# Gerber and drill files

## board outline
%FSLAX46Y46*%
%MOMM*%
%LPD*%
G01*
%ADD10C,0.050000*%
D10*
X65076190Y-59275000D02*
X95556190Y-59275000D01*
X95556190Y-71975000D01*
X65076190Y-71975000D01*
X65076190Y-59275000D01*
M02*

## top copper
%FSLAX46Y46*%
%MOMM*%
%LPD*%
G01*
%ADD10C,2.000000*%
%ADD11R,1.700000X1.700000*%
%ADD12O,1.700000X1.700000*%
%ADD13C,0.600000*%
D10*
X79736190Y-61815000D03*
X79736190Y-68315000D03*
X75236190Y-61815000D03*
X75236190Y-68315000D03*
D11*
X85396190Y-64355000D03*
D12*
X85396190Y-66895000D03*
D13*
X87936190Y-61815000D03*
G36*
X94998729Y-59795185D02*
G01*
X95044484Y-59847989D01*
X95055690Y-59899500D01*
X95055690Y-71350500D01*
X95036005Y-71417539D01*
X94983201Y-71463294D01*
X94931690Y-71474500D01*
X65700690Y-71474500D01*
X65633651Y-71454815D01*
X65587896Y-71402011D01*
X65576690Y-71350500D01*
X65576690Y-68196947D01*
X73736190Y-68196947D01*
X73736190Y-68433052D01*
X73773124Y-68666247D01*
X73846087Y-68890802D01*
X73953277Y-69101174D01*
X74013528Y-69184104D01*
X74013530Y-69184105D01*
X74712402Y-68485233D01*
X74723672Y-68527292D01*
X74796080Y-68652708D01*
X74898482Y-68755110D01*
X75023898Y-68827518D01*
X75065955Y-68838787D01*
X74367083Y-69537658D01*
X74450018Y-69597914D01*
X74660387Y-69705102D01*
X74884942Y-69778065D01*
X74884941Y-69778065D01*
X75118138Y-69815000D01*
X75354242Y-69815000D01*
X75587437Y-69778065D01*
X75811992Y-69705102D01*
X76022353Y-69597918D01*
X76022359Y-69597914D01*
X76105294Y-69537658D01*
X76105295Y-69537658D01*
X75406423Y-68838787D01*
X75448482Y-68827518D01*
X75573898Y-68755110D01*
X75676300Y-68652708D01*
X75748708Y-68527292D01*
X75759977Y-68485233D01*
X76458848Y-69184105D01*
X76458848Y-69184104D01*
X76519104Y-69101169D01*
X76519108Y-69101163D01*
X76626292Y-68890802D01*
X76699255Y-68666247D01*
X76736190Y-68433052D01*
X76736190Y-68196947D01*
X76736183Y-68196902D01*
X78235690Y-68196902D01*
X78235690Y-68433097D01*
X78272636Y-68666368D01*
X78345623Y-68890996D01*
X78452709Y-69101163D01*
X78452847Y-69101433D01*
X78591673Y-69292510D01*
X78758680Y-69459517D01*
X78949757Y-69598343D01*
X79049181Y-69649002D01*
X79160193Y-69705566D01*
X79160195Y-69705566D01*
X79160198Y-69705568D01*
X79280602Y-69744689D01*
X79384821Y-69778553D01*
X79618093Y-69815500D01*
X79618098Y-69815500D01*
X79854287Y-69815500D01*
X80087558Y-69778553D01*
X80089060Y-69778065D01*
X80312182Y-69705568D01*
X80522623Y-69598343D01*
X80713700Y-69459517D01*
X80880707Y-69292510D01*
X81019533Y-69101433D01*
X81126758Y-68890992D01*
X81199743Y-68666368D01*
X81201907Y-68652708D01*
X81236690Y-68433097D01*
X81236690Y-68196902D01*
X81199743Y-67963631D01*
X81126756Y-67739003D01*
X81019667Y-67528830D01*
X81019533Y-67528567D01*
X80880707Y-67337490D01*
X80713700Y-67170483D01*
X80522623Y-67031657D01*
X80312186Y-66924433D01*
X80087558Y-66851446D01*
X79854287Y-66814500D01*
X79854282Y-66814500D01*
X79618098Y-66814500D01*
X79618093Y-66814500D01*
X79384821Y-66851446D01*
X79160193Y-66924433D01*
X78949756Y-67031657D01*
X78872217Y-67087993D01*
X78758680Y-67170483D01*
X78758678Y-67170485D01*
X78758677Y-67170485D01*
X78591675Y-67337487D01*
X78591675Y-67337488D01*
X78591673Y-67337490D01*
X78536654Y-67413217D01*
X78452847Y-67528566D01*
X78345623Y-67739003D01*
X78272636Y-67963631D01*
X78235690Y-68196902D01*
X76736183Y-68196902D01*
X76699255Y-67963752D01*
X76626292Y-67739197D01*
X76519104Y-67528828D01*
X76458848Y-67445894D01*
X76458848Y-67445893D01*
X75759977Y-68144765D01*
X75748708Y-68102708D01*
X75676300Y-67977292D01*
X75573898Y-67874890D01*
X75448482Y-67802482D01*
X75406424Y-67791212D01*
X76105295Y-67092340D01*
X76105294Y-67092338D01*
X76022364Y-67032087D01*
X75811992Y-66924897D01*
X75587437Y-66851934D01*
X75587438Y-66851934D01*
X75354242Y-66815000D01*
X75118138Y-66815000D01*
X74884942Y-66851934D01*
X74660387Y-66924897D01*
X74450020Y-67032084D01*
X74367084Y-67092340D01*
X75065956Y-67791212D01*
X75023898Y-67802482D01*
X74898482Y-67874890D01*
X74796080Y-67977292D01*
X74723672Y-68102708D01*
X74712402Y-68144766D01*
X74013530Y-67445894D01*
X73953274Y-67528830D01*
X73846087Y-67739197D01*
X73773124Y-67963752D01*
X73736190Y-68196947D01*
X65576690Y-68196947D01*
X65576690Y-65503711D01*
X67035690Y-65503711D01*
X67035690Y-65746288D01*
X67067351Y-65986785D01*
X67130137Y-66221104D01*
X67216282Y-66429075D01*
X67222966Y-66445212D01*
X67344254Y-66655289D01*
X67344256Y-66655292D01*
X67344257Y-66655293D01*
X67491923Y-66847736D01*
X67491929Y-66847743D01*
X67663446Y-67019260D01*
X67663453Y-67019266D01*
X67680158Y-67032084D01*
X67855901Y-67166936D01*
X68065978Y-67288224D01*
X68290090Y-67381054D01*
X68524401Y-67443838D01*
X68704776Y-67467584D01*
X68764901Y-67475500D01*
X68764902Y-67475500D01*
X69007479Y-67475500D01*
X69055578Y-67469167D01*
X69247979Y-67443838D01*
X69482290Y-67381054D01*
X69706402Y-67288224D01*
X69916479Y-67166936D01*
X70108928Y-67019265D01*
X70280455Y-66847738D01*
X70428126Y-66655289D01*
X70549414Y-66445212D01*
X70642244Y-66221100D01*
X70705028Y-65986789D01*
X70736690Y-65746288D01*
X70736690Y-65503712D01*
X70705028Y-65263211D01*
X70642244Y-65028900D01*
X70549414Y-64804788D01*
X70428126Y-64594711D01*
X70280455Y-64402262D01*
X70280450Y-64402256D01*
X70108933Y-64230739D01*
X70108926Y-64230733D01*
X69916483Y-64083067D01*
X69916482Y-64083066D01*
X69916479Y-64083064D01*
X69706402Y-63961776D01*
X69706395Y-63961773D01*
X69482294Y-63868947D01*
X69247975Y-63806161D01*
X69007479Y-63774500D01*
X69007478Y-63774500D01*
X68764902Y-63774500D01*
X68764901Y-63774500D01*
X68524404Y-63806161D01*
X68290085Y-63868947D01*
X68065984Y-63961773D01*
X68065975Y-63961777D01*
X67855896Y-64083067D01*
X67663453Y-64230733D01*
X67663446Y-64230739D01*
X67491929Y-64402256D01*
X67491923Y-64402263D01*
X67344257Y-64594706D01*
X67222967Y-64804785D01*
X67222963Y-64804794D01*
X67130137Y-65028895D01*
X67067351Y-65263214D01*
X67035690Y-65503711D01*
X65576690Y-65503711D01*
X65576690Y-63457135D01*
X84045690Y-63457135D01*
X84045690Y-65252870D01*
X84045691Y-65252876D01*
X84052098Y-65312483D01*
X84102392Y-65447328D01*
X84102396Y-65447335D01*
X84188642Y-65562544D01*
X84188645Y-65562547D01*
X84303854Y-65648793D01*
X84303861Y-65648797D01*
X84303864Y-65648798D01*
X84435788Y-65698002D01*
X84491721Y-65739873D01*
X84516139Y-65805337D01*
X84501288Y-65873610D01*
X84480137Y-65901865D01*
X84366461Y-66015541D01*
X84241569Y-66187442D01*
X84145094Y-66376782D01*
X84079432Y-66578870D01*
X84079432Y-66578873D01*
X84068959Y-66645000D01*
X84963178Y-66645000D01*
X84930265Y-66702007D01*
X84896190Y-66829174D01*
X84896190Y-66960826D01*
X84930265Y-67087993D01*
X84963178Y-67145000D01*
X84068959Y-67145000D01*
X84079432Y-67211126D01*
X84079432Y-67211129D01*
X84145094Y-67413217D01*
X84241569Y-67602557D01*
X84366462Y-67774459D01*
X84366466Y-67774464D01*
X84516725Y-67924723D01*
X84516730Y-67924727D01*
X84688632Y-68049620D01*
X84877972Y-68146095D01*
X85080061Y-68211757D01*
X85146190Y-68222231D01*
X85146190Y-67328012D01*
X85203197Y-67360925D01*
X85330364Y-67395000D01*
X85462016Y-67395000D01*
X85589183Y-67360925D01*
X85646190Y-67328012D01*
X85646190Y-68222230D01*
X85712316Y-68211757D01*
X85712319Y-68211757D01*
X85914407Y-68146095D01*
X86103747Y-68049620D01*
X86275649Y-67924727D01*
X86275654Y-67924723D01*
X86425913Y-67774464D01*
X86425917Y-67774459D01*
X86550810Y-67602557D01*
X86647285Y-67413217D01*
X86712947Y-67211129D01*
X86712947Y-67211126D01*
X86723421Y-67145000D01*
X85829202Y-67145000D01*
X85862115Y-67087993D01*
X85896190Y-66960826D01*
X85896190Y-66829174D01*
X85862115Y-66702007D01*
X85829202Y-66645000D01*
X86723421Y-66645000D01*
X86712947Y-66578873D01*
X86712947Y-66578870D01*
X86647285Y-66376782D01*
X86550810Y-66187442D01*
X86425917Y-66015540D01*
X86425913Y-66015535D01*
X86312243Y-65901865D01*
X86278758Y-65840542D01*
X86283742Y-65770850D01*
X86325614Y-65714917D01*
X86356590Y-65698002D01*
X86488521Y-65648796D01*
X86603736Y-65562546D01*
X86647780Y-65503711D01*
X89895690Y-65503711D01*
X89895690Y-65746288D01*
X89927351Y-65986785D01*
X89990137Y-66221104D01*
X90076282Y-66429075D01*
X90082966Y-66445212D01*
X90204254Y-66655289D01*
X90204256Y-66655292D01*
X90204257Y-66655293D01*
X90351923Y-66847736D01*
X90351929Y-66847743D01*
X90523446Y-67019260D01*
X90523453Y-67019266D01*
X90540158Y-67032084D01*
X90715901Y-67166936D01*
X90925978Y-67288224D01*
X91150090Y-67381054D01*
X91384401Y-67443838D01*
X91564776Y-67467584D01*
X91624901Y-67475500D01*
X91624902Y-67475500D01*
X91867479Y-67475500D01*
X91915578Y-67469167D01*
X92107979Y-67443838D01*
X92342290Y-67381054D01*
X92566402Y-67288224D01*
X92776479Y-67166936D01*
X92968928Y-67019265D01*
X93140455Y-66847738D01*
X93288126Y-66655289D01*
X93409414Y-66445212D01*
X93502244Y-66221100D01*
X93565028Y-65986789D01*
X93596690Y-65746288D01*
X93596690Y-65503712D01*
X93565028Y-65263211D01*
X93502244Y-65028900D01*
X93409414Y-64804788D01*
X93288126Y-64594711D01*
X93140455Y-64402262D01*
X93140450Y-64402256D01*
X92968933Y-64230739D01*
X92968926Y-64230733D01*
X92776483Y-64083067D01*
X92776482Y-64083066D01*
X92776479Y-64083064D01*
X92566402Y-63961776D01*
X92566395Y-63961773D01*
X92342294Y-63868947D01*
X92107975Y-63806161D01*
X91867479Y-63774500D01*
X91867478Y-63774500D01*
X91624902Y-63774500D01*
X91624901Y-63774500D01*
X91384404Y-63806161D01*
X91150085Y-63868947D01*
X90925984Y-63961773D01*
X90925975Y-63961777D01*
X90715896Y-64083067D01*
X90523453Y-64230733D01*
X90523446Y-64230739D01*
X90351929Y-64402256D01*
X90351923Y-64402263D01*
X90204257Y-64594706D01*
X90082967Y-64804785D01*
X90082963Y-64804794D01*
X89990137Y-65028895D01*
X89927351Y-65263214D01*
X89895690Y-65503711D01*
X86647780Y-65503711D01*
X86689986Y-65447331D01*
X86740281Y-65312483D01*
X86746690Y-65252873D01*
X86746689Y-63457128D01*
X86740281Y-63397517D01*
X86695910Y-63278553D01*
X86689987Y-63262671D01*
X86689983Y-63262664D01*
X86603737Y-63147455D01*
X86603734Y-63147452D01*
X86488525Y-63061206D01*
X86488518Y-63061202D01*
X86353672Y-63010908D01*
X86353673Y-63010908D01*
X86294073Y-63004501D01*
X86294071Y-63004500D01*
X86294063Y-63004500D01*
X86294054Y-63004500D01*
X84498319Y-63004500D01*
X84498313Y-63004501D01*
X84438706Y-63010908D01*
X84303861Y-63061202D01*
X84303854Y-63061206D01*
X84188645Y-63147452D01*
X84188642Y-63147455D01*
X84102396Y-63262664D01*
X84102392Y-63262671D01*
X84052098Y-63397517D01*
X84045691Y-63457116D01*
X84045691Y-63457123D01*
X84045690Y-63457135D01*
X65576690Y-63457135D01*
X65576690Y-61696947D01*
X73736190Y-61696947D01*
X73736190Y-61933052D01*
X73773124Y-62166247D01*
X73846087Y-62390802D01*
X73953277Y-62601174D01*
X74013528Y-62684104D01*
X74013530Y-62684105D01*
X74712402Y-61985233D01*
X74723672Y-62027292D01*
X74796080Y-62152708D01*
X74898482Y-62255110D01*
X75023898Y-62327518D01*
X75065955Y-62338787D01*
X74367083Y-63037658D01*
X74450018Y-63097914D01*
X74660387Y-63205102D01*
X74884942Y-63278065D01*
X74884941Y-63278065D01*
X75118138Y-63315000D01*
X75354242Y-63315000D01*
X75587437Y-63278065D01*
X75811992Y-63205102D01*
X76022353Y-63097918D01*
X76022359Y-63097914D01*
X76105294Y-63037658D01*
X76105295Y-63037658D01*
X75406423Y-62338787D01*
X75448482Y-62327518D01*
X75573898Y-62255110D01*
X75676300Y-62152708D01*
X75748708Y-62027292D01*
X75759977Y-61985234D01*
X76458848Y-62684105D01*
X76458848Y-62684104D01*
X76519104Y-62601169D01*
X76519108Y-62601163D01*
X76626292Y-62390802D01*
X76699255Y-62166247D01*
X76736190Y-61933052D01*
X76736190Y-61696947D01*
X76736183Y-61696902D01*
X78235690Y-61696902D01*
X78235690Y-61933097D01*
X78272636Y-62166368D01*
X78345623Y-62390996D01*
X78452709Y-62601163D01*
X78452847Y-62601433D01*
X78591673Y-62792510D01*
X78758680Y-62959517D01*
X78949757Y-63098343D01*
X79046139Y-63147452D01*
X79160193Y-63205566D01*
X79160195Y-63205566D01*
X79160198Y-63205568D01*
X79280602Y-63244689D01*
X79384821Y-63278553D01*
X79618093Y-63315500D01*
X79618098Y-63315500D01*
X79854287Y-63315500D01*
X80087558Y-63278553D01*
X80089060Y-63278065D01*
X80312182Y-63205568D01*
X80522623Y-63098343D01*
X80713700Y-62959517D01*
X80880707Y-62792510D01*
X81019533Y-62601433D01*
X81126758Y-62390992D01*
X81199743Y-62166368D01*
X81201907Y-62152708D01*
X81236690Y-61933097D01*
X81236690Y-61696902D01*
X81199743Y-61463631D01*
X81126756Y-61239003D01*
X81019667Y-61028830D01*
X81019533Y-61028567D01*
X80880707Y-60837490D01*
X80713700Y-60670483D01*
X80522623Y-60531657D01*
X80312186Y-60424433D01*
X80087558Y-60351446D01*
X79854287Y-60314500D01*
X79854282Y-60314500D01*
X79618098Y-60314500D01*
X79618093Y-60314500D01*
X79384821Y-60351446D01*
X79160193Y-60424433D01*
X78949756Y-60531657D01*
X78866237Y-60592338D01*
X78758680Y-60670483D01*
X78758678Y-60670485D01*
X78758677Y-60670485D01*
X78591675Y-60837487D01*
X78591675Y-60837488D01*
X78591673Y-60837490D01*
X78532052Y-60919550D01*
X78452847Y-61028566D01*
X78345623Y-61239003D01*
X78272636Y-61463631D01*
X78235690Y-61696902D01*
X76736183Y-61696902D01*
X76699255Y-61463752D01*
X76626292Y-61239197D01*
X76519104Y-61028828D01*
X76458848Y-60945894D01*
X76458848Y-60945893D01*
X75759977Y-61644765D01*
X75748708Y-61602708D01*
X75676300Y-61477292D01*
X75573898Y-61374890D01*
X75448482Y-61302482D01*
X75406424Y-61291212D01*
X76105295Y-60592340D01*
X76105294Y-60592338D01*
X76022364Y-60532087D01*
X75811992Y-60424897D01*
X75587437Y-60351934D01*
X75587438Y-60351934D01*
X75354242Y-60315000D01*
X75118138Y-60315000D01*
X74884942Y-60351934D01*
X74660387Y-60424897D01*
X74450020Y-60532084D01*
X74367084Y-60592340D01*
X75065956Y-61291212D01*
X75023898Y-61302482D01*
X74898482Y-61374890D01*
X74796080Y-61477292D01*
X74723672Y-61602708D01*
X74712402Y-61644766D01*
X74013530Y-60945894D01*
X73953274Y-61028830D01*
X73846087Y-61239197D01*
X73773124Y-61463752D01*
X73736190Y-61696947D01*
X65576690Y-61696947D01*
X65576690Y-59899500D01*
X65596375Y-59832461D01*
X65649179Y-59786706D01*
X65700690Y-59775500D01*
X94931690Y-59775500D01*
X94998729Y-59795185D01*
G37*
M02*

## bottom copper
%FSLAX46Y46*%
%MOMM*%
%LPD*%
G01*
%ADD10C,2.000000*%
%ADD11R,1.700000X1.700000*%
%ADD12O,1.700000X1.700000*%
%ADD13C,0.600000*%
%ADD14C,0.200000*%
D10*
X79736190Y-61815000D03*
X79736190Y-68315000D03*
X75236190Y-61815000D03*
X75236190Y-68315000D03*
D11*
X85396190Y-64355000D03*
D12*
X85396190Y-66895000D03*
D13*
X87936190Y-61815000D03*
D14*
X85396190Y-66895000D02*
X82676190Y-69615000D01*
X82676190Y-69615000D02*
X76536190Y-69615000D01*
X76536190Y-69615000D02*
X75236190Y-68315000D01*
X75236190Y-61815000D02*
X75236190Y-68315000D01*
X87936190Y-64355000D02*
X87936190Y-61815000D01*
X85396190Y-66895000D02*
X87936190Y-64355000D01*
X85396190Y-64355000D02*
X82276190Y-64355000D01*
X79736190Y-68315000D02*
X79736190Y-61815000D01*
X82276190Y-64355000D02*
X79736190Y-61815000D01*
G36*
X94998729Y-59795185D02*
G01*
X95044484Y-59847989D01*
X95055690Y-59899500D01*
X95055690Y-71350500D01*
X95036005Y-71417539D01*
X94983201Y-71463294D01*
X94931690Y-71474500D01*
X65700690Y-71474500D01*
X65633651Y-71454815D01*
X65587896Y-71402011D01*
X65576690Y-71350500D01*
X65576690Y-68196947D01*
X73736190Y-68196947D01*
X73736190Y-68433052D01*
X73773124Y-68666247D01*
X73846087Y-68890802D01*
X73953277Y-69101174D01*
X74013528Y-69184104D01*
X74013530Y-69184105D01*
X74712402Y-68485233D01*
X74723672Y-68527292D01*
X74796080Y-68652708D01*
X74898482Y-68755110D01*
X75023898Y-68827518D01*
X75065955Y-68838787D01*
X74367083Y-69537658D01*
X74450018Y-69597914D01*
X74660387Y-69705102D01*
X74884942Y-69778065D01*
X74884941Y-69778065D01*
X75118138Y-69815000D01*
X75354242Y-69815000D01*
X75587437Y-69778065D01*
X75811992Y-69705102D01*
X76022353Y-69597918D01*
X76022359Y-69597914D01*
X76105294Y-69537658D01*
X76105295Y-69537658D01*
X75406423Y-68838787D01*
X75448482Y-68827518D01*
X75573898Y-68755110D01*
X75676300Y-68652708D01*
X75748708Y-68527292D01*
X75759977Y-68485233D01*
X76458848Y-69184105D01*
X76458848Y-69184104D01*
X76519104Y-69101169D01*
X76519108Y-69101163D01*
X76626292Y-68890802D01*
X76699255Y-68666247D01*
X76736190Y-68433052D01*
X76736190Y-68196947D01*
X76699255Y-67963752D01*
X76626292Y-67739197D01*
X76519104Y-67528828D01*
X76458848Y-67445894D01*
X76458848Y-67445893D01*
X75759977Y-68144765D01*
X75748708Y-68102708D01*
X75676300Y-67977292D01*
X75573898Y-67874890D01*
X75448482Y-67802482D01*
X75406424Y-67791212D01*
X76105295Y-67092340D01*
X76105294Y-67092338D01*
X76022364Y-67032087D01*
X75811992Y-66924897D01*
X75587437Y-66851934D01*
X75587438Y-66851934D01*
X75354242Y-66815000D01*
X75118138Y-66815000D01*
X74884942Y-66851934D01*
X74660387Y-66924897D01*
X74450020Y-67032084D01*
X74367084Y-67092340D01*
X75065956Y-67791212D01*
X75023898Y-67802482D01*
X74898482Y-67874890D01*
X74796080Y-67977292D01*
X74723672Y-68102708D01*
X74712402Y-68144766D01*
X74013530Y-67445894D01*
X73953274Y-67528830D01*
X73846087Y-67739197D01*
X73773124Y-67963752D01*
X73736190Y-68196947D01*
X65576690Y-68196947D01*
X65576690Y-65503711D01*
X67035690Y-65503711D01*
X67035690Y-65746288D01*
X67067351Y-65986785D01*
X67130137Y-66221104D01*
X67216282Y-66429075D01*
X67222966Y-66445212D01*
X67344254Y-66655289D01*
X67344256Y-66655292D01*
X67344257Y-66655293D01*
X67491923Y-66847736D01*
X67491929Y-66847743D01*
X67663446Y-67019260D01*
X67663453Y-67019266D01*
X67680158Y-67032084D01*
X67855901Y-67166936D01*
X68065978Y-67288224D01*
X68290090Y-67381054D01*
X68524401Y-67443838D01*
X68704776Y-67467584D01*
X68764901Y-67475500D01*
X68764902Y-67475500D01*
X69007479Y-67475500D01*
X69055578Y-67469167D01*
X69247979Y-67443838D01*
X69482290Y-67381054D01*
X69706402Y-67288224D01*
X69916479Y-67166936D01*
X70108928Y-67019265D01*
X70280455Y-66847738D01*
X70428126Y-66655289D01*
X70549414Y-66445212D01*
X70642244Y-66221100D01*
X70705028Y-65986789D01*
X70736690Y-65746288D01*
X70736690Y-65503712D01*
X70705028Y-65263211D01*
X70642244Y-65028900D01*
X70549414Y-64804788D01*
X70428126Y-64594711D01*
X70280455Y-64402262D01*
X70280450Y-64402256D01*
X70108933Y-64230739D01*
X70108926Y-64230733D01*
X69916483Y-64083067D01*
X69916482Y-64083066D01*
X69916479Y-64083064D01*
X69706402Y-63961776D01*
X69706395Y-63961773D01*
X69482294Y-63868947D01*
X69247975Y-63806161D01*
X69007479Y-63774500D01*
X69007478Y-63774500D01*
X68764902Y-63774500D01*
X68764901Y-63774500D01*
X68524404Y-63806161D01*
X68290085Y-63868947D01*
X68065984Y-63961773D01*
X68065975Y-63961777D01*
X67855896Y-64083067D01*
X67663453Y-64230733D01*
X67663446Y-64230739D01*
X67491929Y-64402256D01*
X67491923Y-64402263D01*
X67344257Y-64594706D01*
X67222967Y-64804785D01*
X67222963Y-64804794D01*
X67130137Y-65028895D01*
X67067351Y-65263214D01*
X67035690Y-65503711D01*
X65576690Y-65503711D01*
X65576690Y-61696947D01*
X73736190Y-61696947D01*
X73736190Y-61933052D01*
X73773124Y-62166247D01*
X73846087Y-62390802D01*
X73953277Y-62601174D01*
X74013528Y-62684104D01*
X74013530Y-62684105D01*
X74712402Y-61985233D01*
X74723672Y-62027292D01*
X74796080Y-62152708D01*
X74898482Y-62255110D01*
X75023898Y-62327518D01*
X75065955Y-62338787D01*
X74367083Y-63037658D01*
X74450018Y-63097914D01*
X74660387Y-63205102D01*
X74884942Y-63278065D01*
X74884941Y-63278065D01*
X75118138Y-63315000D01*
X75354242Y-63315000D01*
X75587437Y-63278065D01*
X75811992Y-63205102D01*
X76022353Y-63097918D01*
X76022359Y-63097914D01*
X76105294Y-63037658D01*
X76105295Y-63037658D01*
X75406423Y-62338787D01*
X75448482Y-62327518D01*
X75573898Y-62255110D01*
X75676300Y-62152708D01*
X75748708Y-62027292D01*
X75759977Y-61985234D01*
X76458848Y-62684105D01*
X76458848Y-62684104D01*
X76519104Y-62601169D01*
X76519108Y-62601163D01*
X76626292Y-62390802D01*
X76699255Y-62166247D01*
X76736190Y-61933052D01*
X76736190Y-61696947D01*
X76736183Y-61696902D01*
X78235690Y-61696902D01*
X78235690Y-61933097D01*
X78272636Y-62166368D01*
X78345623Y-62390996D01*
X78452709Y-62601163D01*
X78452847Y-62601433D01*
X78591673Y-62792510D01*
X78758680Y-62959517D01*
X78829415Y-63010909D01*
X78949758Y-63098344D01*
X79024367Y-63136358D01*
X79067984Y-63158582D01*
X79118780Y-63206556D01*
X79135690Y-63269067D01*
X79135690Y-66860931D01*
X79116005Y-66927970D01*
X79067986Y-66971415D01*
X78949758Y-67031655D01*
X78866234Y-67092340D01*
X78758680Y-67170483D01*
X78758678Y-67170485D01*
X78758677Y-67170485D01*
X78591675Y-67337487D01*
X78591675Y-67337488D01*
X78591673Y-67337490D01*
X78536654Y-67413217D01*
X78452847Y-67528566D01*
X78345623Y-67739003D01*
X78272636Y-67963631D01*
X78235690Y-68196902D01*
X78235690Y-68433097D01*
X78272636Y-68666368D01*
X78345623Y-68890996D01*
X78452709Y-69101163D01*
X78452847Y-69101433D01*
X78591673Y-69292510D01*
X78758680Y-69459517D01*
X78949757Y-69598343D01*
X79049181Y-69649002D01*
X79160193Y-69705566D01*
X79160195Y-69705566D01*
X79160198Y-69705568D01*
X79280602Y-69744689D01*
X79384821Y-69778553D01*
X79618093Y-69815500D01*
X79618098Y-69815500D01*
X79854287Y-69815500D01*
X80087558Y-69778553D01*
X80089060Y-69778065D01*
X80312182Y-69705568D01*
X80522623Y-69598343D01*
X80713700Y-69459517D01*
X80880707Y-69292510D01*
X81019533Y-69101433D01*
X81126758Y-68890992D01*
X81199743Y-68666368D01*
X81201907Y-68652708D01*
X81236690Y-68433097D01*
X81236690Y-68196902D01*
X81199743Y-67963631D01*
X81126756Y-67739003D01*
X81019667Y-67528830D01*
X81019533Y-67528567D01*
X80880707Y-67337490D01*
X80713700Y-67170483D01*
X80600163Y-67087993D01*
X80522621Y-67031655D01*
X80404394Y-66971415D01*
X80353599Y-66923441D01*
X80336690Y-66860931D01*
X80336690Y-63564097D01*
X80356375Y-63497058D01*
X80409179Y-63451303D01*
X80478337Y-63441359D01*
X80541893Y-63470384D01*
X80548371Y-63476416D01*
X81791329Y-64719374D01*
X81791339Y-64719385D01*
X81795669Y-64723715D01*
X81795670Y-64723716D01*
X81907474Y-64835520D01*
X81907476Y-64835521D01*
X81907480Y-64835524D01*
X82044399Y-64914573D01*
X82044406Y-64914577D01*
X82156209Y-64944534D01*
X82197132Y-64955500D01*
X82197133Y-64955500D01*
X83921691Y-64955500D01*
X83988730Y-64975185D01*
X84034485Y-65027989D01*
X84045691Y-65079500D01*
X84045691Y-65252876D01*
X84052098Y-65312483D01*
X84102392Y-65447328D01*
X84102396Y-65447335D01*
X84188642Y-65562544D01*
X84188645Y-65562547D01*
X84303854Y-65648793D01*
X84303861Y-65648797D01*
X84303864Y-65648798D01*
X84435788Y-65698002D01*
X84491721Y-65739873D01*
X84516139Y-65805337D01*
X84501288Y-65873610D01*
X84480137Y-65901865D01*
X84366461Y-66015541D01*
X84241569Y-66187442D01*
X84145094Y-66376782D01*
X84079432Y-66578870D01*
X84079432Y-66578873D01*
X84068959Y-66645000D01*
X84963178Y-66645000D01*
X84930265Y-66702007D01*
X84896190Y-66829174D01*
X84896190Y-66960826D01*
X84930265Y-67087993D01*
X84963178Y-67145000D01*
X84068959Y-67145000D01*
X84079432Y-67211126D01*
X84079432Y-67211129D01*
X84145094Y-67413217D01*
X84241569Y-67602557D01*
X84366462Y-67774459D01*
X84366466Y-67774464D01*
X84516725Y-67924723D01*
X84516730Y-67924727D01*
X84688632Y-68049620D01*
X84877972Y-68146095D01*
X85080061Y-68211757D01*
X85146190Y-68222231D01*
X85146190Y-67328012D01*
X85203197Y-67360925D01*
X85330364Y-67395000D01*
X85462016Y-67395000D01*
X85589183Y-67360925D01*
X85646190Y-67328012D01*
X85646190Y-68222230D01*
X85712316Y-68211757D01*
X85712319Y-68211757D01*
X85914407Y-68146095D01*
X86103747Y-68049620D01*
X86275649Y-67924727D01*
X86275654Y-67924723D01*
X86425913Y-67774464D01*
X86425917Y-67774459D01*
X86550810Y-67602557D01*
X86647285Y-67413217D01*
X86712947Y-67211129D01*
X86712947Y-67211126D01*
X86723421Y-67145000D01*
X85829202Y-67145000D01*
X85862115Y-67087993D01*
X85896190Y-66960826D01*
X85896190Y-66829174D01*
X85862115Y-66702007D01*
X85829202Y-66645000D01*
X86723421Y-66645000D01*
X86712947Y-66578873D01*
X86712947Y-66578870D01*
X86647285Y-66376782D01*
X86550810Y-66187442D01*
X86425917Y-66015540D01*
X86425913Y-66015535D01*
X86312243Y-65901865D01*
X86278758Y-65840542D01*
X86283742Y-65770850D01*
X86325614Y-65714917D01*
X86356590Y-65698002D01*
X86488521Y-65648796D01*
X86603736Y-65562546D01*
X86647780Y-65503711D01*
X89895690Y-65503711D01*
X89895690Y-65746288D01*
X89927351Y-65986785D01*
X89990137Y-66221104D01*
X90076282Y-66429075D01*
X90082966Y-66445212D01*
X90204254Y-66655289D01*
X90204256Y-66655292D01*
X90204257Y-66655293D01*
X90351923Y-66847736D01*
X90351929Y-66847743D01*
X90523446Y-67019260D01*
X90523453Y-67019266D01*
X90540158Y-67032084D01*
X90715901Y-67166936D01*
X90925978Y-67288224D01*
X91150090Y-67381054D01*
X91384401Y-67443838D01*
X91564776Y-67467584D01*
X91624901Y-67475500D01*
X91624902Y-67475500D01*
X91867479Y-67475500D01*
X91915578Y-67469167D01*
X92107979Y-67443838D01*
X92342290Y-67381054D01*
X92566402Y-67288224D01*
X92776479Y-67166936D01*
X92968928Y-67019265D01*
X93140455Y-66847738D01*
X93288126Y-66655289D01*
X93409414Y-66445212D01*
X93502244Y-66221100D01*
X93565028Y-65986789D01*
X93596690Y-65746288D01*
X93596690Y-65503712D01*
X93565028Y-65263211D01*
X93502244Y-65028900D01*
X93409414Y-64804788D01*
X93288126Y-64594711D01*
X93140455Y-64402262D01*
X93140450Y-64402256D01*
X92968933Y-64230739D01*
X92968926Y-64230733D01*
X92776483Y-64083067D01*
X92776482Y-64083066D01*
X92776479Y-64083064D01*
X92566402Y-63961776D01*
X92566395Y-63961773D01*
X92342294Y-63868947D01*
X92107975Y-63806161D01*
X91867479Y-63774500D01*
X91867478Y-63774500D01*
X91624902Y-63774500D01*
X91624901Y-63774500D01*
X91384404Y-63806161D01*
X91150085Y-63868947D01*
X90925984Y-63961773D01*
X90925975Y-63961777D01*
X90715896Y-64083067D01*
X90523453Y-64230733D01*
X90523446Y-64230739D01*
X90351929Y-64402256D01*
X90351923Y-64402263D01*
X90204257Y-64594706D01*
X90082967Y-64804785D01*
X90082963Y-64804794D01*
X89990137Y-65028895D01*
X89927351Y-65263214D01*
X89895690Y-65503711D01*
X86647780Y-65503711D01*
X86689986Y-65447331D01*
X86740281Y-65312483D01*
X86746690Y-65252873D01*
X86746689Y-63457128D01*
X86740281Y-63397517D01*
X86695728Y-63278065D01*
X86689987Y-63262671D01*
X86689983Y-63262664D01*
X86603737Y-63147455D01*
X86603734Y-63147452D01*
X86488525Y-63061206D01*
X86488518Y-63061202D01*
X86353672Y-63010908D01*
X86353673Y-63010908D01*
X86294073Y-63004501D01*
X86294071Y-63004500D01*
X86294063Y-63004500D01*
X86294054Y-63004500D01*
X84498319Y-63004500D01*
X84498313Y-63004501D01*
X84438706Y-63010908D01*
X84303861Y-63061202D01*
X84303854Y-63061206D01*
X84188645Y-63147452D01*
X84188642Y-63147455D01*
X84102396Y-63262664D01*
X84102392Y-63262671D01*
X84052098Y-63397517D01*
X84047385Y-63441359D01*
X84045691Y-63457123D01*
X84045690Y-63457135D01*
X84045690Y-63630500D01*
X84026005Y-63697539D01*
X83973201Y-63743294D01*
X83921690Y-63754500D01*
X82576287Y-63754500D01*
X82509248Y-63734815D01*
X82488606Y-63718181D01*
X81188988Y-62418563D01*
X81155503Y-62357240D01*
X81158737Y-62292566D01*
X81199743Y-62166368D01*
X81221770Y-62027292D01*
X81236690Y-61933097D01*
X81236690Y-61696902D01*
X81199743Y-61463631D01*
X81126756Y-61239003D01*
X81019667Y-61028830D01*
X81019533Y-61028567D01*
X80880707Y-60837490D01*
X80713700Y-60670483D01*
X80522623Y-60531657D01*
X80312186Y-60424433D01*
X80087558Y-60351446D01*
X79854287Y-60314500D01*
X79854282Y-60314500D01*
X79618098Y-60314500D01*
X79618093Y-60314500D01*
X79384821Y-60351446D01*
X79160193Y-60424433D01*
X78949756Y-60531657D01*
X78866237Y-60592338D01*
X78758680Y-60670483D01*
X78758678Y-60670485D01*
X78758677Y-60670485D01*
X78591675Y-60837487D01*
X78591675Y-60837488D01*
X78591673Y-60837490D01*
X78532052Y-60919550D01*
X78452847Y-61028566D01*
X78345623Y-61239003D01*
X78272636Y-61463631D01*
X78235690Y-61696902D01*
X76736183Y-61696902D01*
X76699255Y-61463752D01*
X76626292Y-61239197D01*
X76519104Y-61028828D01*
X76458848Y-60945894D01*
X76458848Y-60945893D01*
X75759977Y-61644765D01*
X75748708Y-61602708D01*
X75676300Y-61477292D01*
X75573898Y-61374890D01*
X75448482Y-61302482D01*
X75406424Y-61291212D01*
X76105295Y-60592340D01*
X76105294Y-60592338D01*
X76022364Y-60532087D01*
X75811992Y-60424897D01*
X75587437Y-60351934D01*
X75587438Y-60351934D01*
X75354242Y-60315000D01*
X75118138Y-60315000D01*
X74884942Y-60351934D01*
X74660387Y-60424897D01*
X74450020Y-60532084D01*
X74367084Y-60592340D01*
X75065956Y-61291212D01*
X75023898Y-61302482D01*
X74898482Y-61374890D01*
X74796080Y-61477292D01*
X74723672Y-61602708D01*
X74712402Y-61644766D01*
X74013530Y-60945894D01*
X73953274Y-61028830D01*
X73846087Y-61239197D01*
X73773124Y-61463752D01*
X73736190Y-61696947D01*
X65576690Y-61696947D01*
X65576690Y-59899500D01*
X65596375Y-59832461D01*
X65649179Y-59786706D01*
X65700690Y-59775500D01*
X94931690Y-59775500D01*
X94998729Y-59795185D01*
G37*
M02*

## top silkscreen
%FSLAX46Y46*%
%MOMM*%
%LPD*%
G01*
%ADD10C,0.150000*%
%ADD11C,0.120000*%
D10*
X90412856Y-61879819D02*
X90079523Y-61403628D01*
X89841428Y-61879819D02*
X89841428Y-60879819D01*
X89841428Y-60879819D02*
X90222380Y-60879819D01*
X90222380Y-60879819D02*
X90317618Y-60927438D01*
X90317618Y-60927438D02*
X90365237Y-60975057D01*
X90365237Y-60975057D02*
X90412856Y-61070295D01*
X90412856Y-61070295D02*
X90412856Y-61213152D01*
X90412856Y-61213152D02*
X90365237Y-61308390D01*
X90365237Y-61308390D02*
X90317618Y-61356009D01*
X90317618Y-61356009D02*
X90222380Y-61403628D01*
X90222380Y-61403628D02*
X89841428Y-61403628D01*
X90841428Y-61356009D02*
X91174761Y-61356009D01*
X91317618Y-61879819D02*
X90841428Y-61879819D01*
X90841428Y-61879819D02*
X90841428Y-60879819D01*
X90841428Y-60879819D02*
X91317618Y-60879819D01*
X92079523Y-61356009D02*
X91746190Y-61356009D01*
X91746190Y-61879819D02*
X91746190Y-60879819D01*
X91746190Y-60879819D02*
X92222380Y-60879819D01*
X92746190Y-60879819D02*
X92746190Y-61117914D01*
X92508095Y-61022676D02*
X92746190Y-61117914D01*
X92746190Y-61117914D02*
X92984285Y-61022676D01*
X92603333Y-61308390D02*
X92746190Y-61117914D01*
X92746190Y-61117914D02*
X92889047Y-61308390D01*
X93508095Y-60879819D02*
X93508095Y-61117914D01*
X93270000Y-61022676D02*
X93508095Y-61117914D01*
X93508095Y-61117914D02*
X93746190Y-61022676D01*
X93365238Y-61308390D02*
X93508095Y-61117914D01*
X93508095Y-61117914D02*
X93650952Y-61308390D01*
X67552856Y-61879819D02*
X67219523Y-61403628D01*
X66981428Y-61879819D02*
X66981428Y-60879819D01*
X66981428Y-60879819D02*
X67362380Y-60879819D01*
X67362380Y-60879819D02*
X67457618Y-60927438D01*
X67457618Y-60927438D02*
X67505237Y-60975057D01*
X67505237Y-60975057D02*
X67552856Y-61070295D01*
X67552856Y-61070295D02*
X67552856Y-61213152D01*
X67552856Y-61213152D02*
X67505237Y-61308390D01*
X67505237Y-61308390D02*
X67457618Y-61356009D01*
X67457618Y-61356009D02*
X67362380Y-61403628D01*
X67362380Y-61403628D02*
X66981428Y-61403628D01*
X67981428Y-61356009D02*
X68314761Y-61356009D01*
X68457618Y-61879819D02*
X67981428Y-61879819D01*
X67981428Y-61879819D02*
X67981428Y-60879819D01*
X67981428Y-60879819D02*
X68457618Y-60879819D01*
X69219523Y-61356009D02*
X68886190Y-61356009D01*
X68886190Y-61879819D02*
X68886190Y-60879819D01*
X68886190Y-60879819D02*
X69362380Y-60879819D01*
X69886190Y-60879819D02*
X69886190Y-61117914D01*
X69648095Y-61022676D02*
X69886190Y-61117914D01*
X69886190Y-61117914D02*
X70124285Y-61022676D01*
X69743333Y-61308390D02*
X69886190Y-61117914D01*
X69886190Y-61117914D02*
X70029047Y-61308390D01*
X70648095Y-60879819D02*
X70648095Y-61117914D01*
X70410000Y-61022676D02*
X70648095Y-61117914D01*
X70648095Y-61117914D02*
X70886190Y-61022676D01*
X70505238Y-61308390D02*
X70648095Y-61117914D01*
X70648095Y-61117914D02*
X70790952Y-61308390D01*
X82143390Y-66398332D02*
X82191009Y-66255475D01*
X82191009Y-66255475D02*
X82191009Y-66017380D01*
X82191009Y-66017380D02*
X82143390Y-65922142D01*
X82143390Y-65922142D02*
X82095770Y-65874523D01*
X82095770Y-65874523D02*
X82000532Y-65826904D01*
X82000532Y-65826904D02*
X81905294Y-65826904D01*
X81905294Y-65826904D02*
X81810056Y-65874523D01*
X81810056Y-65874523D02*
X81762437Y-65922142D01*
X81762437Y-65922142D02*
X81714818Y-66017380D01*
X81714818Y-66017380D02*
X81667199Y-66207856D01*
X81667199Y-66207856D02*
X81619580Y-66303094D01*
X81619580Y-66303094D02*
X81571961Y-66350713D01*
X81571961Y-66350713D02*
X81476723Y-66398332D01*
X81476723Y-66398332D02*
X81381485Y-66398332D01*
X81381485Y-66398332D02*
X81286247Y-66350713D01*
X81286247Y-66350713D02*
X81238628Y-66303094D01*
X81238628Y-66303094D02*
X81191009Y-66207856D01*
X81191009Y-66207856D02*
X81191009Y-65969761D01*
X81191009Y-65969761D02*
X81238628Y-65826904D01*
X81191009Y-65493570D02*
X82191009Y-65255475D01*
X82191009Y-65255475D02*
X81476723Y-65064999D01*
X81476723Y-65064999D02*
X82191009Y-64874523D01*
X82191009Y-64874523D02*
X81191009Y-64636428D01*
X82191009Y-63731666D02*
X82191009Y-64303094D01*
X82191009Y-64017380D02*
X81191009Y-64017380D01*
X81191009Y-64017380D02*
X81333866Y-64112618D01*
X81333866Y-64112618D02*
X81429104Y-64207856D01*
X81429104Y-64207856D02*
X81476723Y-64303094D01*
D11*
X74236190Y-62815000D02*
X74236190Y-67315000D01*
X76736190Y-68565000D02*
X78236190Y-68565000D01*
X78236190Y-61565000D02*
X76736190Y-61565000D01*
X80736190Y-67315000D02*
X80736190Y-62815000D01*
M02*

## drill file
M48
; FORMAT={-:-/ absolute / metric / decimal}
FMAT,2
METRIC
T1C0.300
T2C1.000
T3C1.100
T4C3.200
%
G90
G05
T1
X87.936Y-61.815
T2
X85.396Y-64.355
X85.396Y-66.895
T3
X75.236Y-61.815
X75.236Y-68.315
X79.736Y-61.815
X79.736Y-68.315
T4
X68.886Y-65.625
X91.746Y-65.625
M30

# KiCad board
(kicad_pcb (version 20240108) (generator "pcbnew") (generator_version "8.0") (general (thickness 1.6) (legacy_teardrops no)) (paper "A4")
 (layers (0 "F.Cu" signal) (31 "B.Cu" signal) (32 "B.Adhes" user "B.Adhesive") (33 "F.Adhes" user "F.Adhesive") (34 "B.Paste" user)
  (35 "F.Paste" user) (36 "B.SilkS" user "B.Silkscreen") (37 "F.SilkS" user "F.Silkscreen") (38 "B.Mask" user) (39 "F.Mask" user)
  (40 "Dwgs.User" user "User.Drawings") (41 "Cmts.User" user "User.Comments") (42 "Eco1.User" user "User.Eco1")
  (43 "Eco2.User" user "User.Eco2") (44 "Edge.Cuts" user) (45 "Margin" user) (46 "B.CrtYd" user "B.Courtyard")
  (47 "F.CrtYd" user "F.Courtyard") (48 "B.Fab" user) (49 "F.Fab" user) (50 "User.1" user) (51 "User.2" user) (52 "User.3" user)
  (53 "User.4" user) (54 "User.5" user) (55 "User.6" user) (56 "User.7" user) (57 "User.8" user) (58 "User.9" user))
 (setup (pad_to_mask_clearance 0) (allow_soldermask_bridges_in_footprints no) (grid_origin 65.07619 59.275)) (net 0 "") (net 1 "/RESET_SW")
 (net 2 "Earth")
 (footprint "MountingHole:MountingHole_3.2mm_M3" (layer "F.Cu") (at 91.74619 65.625)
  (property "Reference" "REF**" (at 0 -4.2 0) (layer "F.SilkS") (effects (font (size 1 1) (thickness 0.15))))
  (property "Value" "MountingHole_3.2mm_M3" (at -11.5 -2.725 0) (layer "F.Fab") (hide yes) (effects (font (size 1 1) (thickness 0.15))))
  (pad "" np_thru_hole circle (at 0 0) (size 3.2 3.2) (drill 3.2) (layers "*.Cu" "*.Mask")))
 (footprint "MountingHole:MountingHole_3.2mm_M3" (layer "F.Cu") (at 68.88619 65.625)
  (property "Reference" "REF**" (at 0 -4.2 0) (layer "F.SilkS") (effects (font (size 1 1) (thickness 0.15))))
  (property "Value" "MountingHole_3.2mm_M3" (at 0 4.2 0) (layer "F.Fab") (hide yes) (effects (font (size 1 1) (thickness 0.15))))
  (pad "" np_thru_hole circle (at 0 0) (size 3.2 3.2) (drill 3.2) (layers "*.Cu" "*.Mask")))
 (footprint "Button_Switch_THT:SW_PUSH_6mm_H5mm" (layer "F.Cu") (at 79.73619 61.815 -90)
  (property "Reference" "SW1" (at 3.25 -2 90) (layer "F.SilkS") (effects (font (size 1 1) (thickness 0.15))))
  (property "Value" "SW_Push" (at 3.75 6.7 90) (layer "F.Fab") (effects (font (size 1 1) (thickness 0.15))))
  (fp_line (start 1 5.5) (end 5.5 5.5) (stroke (width 0.12) (type solid)) (layer "F.SilkS"))
  (fp_line (start 6.75 3) (end 6.75 1.5) (stroke (width 0.12) (type solid)) (layer "F.SilkS"))
  (fp_line (start -0.25 1.5) (end -0.25 3) (stroke (width 0.12) (type solid)) (layer "F.SilkS"))
  (fp_line (start 5.5 -1) (end 1 -1) (stroke (width 0.12) (type solid)) (layer "F.SilkS"))
  (pad "1" thru_hole circle (at 0 0) (size 2 2) (drill 1.1) (layers "*.Cu" "*.Mask") (remove_unused_layers no) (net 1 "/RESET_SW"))
  (pad "1" thru_hole circle (at 6.5 0) (size 2 2) (drill 1.1) (layers "*.Cu" "*.Mask") (remove_unused_layers no) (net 1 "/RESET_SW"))
  (pad "2" thru_hole circle (at 0 4.5) (size 2 2) (drill 1.1) (layers "*.Cu" "*.Mask") (remove_unused_layers no) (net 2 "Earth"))
  (pad "2" thru_hole circle (at 6.5 4.5) (size 2 2) (drill 1.1) (layers "*.Cu" "*.Mask") (remove_unused_layers no) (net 2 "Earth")))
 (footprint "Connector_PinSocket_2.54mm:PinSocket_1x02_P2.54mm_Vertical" (layer "B.Cu") (at 85.39619 64.355 180)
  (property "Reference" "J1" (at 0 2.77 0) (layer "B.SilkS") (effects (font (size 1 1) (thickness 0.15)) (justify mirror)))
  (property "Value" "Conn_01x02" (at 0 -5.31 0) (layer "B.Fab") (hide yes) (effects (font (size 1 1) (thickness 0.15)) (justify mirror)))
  (pad "1" thru_hole rect (at 0 0 180) (size 1.7 1.7) (drill 1) (layers "*.Cu" "*.Mask") (remove_unused_layers no) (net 1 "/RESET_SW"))
  (pad "2" thru_hole oval (at 0 -2.54 180) (size 1.7 1.7) (drill 1) (layers "*.Cu" "*.Mask") (remove_unused_layers no) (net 2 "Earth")))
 (gr_rect (start 65.07619 59.275) (end 95.55619 71.975) (stroke (width 0.05) (type default)) (fill none) (layer "Edge.Cuts"))
 (via (at 87.93619 61.815) (size 0.6) (drill 0.3) (layers "F.Cu" "B.Cu") (free yes) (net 2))
 (segment (start 85.39619 66.895) (end 82.67619 69.615) (width 0.2) (layer "B.Cu") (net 2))
 (segment (start 82.67619 69.615) (end 76.53619 69.615) (width 0.2) (layer "B.Cu") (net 2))
 (segment (start 76.53619 69.615) (end 75.23619 68.315) (width 0.2) (layer "B.Cu") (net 2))
 (segment (start 75.23619 61.815) (end 75.23619 68.315) (width 0.2) (layer "B.Cu") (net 2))
 (segment (start 87.93619 64.355) (end 87.93619 61.815) (width 0.2) (layer "B.Cu") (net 2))
 (segment (start 85.39619 66.895) (end 87.93619 64.355) (width 0.2) (layer "B.Cu") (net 2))
 (segment (start 85.39619 64.355) (end 82.27619 64.355) (width 0.2) (layer "B.Cu") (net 1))
 (segment (start 79.73619 68.315) (end 79.73619 61.815) (width 0.2) (layer "B.Cu") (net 1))
 (segment (start 82.27619 64.355) (end 79.73619 61.815) (width 0.2) (layer "B.Cu") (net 1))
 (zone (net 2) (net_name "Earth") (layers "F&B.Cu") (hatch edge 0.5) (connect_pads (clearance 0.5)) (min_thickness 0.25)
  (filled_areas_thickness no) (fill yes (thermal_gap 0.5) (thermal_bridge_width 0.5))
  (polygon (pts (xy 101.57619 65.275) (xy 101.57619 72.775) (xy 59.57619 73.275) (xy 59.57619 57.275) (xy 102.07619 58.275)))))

